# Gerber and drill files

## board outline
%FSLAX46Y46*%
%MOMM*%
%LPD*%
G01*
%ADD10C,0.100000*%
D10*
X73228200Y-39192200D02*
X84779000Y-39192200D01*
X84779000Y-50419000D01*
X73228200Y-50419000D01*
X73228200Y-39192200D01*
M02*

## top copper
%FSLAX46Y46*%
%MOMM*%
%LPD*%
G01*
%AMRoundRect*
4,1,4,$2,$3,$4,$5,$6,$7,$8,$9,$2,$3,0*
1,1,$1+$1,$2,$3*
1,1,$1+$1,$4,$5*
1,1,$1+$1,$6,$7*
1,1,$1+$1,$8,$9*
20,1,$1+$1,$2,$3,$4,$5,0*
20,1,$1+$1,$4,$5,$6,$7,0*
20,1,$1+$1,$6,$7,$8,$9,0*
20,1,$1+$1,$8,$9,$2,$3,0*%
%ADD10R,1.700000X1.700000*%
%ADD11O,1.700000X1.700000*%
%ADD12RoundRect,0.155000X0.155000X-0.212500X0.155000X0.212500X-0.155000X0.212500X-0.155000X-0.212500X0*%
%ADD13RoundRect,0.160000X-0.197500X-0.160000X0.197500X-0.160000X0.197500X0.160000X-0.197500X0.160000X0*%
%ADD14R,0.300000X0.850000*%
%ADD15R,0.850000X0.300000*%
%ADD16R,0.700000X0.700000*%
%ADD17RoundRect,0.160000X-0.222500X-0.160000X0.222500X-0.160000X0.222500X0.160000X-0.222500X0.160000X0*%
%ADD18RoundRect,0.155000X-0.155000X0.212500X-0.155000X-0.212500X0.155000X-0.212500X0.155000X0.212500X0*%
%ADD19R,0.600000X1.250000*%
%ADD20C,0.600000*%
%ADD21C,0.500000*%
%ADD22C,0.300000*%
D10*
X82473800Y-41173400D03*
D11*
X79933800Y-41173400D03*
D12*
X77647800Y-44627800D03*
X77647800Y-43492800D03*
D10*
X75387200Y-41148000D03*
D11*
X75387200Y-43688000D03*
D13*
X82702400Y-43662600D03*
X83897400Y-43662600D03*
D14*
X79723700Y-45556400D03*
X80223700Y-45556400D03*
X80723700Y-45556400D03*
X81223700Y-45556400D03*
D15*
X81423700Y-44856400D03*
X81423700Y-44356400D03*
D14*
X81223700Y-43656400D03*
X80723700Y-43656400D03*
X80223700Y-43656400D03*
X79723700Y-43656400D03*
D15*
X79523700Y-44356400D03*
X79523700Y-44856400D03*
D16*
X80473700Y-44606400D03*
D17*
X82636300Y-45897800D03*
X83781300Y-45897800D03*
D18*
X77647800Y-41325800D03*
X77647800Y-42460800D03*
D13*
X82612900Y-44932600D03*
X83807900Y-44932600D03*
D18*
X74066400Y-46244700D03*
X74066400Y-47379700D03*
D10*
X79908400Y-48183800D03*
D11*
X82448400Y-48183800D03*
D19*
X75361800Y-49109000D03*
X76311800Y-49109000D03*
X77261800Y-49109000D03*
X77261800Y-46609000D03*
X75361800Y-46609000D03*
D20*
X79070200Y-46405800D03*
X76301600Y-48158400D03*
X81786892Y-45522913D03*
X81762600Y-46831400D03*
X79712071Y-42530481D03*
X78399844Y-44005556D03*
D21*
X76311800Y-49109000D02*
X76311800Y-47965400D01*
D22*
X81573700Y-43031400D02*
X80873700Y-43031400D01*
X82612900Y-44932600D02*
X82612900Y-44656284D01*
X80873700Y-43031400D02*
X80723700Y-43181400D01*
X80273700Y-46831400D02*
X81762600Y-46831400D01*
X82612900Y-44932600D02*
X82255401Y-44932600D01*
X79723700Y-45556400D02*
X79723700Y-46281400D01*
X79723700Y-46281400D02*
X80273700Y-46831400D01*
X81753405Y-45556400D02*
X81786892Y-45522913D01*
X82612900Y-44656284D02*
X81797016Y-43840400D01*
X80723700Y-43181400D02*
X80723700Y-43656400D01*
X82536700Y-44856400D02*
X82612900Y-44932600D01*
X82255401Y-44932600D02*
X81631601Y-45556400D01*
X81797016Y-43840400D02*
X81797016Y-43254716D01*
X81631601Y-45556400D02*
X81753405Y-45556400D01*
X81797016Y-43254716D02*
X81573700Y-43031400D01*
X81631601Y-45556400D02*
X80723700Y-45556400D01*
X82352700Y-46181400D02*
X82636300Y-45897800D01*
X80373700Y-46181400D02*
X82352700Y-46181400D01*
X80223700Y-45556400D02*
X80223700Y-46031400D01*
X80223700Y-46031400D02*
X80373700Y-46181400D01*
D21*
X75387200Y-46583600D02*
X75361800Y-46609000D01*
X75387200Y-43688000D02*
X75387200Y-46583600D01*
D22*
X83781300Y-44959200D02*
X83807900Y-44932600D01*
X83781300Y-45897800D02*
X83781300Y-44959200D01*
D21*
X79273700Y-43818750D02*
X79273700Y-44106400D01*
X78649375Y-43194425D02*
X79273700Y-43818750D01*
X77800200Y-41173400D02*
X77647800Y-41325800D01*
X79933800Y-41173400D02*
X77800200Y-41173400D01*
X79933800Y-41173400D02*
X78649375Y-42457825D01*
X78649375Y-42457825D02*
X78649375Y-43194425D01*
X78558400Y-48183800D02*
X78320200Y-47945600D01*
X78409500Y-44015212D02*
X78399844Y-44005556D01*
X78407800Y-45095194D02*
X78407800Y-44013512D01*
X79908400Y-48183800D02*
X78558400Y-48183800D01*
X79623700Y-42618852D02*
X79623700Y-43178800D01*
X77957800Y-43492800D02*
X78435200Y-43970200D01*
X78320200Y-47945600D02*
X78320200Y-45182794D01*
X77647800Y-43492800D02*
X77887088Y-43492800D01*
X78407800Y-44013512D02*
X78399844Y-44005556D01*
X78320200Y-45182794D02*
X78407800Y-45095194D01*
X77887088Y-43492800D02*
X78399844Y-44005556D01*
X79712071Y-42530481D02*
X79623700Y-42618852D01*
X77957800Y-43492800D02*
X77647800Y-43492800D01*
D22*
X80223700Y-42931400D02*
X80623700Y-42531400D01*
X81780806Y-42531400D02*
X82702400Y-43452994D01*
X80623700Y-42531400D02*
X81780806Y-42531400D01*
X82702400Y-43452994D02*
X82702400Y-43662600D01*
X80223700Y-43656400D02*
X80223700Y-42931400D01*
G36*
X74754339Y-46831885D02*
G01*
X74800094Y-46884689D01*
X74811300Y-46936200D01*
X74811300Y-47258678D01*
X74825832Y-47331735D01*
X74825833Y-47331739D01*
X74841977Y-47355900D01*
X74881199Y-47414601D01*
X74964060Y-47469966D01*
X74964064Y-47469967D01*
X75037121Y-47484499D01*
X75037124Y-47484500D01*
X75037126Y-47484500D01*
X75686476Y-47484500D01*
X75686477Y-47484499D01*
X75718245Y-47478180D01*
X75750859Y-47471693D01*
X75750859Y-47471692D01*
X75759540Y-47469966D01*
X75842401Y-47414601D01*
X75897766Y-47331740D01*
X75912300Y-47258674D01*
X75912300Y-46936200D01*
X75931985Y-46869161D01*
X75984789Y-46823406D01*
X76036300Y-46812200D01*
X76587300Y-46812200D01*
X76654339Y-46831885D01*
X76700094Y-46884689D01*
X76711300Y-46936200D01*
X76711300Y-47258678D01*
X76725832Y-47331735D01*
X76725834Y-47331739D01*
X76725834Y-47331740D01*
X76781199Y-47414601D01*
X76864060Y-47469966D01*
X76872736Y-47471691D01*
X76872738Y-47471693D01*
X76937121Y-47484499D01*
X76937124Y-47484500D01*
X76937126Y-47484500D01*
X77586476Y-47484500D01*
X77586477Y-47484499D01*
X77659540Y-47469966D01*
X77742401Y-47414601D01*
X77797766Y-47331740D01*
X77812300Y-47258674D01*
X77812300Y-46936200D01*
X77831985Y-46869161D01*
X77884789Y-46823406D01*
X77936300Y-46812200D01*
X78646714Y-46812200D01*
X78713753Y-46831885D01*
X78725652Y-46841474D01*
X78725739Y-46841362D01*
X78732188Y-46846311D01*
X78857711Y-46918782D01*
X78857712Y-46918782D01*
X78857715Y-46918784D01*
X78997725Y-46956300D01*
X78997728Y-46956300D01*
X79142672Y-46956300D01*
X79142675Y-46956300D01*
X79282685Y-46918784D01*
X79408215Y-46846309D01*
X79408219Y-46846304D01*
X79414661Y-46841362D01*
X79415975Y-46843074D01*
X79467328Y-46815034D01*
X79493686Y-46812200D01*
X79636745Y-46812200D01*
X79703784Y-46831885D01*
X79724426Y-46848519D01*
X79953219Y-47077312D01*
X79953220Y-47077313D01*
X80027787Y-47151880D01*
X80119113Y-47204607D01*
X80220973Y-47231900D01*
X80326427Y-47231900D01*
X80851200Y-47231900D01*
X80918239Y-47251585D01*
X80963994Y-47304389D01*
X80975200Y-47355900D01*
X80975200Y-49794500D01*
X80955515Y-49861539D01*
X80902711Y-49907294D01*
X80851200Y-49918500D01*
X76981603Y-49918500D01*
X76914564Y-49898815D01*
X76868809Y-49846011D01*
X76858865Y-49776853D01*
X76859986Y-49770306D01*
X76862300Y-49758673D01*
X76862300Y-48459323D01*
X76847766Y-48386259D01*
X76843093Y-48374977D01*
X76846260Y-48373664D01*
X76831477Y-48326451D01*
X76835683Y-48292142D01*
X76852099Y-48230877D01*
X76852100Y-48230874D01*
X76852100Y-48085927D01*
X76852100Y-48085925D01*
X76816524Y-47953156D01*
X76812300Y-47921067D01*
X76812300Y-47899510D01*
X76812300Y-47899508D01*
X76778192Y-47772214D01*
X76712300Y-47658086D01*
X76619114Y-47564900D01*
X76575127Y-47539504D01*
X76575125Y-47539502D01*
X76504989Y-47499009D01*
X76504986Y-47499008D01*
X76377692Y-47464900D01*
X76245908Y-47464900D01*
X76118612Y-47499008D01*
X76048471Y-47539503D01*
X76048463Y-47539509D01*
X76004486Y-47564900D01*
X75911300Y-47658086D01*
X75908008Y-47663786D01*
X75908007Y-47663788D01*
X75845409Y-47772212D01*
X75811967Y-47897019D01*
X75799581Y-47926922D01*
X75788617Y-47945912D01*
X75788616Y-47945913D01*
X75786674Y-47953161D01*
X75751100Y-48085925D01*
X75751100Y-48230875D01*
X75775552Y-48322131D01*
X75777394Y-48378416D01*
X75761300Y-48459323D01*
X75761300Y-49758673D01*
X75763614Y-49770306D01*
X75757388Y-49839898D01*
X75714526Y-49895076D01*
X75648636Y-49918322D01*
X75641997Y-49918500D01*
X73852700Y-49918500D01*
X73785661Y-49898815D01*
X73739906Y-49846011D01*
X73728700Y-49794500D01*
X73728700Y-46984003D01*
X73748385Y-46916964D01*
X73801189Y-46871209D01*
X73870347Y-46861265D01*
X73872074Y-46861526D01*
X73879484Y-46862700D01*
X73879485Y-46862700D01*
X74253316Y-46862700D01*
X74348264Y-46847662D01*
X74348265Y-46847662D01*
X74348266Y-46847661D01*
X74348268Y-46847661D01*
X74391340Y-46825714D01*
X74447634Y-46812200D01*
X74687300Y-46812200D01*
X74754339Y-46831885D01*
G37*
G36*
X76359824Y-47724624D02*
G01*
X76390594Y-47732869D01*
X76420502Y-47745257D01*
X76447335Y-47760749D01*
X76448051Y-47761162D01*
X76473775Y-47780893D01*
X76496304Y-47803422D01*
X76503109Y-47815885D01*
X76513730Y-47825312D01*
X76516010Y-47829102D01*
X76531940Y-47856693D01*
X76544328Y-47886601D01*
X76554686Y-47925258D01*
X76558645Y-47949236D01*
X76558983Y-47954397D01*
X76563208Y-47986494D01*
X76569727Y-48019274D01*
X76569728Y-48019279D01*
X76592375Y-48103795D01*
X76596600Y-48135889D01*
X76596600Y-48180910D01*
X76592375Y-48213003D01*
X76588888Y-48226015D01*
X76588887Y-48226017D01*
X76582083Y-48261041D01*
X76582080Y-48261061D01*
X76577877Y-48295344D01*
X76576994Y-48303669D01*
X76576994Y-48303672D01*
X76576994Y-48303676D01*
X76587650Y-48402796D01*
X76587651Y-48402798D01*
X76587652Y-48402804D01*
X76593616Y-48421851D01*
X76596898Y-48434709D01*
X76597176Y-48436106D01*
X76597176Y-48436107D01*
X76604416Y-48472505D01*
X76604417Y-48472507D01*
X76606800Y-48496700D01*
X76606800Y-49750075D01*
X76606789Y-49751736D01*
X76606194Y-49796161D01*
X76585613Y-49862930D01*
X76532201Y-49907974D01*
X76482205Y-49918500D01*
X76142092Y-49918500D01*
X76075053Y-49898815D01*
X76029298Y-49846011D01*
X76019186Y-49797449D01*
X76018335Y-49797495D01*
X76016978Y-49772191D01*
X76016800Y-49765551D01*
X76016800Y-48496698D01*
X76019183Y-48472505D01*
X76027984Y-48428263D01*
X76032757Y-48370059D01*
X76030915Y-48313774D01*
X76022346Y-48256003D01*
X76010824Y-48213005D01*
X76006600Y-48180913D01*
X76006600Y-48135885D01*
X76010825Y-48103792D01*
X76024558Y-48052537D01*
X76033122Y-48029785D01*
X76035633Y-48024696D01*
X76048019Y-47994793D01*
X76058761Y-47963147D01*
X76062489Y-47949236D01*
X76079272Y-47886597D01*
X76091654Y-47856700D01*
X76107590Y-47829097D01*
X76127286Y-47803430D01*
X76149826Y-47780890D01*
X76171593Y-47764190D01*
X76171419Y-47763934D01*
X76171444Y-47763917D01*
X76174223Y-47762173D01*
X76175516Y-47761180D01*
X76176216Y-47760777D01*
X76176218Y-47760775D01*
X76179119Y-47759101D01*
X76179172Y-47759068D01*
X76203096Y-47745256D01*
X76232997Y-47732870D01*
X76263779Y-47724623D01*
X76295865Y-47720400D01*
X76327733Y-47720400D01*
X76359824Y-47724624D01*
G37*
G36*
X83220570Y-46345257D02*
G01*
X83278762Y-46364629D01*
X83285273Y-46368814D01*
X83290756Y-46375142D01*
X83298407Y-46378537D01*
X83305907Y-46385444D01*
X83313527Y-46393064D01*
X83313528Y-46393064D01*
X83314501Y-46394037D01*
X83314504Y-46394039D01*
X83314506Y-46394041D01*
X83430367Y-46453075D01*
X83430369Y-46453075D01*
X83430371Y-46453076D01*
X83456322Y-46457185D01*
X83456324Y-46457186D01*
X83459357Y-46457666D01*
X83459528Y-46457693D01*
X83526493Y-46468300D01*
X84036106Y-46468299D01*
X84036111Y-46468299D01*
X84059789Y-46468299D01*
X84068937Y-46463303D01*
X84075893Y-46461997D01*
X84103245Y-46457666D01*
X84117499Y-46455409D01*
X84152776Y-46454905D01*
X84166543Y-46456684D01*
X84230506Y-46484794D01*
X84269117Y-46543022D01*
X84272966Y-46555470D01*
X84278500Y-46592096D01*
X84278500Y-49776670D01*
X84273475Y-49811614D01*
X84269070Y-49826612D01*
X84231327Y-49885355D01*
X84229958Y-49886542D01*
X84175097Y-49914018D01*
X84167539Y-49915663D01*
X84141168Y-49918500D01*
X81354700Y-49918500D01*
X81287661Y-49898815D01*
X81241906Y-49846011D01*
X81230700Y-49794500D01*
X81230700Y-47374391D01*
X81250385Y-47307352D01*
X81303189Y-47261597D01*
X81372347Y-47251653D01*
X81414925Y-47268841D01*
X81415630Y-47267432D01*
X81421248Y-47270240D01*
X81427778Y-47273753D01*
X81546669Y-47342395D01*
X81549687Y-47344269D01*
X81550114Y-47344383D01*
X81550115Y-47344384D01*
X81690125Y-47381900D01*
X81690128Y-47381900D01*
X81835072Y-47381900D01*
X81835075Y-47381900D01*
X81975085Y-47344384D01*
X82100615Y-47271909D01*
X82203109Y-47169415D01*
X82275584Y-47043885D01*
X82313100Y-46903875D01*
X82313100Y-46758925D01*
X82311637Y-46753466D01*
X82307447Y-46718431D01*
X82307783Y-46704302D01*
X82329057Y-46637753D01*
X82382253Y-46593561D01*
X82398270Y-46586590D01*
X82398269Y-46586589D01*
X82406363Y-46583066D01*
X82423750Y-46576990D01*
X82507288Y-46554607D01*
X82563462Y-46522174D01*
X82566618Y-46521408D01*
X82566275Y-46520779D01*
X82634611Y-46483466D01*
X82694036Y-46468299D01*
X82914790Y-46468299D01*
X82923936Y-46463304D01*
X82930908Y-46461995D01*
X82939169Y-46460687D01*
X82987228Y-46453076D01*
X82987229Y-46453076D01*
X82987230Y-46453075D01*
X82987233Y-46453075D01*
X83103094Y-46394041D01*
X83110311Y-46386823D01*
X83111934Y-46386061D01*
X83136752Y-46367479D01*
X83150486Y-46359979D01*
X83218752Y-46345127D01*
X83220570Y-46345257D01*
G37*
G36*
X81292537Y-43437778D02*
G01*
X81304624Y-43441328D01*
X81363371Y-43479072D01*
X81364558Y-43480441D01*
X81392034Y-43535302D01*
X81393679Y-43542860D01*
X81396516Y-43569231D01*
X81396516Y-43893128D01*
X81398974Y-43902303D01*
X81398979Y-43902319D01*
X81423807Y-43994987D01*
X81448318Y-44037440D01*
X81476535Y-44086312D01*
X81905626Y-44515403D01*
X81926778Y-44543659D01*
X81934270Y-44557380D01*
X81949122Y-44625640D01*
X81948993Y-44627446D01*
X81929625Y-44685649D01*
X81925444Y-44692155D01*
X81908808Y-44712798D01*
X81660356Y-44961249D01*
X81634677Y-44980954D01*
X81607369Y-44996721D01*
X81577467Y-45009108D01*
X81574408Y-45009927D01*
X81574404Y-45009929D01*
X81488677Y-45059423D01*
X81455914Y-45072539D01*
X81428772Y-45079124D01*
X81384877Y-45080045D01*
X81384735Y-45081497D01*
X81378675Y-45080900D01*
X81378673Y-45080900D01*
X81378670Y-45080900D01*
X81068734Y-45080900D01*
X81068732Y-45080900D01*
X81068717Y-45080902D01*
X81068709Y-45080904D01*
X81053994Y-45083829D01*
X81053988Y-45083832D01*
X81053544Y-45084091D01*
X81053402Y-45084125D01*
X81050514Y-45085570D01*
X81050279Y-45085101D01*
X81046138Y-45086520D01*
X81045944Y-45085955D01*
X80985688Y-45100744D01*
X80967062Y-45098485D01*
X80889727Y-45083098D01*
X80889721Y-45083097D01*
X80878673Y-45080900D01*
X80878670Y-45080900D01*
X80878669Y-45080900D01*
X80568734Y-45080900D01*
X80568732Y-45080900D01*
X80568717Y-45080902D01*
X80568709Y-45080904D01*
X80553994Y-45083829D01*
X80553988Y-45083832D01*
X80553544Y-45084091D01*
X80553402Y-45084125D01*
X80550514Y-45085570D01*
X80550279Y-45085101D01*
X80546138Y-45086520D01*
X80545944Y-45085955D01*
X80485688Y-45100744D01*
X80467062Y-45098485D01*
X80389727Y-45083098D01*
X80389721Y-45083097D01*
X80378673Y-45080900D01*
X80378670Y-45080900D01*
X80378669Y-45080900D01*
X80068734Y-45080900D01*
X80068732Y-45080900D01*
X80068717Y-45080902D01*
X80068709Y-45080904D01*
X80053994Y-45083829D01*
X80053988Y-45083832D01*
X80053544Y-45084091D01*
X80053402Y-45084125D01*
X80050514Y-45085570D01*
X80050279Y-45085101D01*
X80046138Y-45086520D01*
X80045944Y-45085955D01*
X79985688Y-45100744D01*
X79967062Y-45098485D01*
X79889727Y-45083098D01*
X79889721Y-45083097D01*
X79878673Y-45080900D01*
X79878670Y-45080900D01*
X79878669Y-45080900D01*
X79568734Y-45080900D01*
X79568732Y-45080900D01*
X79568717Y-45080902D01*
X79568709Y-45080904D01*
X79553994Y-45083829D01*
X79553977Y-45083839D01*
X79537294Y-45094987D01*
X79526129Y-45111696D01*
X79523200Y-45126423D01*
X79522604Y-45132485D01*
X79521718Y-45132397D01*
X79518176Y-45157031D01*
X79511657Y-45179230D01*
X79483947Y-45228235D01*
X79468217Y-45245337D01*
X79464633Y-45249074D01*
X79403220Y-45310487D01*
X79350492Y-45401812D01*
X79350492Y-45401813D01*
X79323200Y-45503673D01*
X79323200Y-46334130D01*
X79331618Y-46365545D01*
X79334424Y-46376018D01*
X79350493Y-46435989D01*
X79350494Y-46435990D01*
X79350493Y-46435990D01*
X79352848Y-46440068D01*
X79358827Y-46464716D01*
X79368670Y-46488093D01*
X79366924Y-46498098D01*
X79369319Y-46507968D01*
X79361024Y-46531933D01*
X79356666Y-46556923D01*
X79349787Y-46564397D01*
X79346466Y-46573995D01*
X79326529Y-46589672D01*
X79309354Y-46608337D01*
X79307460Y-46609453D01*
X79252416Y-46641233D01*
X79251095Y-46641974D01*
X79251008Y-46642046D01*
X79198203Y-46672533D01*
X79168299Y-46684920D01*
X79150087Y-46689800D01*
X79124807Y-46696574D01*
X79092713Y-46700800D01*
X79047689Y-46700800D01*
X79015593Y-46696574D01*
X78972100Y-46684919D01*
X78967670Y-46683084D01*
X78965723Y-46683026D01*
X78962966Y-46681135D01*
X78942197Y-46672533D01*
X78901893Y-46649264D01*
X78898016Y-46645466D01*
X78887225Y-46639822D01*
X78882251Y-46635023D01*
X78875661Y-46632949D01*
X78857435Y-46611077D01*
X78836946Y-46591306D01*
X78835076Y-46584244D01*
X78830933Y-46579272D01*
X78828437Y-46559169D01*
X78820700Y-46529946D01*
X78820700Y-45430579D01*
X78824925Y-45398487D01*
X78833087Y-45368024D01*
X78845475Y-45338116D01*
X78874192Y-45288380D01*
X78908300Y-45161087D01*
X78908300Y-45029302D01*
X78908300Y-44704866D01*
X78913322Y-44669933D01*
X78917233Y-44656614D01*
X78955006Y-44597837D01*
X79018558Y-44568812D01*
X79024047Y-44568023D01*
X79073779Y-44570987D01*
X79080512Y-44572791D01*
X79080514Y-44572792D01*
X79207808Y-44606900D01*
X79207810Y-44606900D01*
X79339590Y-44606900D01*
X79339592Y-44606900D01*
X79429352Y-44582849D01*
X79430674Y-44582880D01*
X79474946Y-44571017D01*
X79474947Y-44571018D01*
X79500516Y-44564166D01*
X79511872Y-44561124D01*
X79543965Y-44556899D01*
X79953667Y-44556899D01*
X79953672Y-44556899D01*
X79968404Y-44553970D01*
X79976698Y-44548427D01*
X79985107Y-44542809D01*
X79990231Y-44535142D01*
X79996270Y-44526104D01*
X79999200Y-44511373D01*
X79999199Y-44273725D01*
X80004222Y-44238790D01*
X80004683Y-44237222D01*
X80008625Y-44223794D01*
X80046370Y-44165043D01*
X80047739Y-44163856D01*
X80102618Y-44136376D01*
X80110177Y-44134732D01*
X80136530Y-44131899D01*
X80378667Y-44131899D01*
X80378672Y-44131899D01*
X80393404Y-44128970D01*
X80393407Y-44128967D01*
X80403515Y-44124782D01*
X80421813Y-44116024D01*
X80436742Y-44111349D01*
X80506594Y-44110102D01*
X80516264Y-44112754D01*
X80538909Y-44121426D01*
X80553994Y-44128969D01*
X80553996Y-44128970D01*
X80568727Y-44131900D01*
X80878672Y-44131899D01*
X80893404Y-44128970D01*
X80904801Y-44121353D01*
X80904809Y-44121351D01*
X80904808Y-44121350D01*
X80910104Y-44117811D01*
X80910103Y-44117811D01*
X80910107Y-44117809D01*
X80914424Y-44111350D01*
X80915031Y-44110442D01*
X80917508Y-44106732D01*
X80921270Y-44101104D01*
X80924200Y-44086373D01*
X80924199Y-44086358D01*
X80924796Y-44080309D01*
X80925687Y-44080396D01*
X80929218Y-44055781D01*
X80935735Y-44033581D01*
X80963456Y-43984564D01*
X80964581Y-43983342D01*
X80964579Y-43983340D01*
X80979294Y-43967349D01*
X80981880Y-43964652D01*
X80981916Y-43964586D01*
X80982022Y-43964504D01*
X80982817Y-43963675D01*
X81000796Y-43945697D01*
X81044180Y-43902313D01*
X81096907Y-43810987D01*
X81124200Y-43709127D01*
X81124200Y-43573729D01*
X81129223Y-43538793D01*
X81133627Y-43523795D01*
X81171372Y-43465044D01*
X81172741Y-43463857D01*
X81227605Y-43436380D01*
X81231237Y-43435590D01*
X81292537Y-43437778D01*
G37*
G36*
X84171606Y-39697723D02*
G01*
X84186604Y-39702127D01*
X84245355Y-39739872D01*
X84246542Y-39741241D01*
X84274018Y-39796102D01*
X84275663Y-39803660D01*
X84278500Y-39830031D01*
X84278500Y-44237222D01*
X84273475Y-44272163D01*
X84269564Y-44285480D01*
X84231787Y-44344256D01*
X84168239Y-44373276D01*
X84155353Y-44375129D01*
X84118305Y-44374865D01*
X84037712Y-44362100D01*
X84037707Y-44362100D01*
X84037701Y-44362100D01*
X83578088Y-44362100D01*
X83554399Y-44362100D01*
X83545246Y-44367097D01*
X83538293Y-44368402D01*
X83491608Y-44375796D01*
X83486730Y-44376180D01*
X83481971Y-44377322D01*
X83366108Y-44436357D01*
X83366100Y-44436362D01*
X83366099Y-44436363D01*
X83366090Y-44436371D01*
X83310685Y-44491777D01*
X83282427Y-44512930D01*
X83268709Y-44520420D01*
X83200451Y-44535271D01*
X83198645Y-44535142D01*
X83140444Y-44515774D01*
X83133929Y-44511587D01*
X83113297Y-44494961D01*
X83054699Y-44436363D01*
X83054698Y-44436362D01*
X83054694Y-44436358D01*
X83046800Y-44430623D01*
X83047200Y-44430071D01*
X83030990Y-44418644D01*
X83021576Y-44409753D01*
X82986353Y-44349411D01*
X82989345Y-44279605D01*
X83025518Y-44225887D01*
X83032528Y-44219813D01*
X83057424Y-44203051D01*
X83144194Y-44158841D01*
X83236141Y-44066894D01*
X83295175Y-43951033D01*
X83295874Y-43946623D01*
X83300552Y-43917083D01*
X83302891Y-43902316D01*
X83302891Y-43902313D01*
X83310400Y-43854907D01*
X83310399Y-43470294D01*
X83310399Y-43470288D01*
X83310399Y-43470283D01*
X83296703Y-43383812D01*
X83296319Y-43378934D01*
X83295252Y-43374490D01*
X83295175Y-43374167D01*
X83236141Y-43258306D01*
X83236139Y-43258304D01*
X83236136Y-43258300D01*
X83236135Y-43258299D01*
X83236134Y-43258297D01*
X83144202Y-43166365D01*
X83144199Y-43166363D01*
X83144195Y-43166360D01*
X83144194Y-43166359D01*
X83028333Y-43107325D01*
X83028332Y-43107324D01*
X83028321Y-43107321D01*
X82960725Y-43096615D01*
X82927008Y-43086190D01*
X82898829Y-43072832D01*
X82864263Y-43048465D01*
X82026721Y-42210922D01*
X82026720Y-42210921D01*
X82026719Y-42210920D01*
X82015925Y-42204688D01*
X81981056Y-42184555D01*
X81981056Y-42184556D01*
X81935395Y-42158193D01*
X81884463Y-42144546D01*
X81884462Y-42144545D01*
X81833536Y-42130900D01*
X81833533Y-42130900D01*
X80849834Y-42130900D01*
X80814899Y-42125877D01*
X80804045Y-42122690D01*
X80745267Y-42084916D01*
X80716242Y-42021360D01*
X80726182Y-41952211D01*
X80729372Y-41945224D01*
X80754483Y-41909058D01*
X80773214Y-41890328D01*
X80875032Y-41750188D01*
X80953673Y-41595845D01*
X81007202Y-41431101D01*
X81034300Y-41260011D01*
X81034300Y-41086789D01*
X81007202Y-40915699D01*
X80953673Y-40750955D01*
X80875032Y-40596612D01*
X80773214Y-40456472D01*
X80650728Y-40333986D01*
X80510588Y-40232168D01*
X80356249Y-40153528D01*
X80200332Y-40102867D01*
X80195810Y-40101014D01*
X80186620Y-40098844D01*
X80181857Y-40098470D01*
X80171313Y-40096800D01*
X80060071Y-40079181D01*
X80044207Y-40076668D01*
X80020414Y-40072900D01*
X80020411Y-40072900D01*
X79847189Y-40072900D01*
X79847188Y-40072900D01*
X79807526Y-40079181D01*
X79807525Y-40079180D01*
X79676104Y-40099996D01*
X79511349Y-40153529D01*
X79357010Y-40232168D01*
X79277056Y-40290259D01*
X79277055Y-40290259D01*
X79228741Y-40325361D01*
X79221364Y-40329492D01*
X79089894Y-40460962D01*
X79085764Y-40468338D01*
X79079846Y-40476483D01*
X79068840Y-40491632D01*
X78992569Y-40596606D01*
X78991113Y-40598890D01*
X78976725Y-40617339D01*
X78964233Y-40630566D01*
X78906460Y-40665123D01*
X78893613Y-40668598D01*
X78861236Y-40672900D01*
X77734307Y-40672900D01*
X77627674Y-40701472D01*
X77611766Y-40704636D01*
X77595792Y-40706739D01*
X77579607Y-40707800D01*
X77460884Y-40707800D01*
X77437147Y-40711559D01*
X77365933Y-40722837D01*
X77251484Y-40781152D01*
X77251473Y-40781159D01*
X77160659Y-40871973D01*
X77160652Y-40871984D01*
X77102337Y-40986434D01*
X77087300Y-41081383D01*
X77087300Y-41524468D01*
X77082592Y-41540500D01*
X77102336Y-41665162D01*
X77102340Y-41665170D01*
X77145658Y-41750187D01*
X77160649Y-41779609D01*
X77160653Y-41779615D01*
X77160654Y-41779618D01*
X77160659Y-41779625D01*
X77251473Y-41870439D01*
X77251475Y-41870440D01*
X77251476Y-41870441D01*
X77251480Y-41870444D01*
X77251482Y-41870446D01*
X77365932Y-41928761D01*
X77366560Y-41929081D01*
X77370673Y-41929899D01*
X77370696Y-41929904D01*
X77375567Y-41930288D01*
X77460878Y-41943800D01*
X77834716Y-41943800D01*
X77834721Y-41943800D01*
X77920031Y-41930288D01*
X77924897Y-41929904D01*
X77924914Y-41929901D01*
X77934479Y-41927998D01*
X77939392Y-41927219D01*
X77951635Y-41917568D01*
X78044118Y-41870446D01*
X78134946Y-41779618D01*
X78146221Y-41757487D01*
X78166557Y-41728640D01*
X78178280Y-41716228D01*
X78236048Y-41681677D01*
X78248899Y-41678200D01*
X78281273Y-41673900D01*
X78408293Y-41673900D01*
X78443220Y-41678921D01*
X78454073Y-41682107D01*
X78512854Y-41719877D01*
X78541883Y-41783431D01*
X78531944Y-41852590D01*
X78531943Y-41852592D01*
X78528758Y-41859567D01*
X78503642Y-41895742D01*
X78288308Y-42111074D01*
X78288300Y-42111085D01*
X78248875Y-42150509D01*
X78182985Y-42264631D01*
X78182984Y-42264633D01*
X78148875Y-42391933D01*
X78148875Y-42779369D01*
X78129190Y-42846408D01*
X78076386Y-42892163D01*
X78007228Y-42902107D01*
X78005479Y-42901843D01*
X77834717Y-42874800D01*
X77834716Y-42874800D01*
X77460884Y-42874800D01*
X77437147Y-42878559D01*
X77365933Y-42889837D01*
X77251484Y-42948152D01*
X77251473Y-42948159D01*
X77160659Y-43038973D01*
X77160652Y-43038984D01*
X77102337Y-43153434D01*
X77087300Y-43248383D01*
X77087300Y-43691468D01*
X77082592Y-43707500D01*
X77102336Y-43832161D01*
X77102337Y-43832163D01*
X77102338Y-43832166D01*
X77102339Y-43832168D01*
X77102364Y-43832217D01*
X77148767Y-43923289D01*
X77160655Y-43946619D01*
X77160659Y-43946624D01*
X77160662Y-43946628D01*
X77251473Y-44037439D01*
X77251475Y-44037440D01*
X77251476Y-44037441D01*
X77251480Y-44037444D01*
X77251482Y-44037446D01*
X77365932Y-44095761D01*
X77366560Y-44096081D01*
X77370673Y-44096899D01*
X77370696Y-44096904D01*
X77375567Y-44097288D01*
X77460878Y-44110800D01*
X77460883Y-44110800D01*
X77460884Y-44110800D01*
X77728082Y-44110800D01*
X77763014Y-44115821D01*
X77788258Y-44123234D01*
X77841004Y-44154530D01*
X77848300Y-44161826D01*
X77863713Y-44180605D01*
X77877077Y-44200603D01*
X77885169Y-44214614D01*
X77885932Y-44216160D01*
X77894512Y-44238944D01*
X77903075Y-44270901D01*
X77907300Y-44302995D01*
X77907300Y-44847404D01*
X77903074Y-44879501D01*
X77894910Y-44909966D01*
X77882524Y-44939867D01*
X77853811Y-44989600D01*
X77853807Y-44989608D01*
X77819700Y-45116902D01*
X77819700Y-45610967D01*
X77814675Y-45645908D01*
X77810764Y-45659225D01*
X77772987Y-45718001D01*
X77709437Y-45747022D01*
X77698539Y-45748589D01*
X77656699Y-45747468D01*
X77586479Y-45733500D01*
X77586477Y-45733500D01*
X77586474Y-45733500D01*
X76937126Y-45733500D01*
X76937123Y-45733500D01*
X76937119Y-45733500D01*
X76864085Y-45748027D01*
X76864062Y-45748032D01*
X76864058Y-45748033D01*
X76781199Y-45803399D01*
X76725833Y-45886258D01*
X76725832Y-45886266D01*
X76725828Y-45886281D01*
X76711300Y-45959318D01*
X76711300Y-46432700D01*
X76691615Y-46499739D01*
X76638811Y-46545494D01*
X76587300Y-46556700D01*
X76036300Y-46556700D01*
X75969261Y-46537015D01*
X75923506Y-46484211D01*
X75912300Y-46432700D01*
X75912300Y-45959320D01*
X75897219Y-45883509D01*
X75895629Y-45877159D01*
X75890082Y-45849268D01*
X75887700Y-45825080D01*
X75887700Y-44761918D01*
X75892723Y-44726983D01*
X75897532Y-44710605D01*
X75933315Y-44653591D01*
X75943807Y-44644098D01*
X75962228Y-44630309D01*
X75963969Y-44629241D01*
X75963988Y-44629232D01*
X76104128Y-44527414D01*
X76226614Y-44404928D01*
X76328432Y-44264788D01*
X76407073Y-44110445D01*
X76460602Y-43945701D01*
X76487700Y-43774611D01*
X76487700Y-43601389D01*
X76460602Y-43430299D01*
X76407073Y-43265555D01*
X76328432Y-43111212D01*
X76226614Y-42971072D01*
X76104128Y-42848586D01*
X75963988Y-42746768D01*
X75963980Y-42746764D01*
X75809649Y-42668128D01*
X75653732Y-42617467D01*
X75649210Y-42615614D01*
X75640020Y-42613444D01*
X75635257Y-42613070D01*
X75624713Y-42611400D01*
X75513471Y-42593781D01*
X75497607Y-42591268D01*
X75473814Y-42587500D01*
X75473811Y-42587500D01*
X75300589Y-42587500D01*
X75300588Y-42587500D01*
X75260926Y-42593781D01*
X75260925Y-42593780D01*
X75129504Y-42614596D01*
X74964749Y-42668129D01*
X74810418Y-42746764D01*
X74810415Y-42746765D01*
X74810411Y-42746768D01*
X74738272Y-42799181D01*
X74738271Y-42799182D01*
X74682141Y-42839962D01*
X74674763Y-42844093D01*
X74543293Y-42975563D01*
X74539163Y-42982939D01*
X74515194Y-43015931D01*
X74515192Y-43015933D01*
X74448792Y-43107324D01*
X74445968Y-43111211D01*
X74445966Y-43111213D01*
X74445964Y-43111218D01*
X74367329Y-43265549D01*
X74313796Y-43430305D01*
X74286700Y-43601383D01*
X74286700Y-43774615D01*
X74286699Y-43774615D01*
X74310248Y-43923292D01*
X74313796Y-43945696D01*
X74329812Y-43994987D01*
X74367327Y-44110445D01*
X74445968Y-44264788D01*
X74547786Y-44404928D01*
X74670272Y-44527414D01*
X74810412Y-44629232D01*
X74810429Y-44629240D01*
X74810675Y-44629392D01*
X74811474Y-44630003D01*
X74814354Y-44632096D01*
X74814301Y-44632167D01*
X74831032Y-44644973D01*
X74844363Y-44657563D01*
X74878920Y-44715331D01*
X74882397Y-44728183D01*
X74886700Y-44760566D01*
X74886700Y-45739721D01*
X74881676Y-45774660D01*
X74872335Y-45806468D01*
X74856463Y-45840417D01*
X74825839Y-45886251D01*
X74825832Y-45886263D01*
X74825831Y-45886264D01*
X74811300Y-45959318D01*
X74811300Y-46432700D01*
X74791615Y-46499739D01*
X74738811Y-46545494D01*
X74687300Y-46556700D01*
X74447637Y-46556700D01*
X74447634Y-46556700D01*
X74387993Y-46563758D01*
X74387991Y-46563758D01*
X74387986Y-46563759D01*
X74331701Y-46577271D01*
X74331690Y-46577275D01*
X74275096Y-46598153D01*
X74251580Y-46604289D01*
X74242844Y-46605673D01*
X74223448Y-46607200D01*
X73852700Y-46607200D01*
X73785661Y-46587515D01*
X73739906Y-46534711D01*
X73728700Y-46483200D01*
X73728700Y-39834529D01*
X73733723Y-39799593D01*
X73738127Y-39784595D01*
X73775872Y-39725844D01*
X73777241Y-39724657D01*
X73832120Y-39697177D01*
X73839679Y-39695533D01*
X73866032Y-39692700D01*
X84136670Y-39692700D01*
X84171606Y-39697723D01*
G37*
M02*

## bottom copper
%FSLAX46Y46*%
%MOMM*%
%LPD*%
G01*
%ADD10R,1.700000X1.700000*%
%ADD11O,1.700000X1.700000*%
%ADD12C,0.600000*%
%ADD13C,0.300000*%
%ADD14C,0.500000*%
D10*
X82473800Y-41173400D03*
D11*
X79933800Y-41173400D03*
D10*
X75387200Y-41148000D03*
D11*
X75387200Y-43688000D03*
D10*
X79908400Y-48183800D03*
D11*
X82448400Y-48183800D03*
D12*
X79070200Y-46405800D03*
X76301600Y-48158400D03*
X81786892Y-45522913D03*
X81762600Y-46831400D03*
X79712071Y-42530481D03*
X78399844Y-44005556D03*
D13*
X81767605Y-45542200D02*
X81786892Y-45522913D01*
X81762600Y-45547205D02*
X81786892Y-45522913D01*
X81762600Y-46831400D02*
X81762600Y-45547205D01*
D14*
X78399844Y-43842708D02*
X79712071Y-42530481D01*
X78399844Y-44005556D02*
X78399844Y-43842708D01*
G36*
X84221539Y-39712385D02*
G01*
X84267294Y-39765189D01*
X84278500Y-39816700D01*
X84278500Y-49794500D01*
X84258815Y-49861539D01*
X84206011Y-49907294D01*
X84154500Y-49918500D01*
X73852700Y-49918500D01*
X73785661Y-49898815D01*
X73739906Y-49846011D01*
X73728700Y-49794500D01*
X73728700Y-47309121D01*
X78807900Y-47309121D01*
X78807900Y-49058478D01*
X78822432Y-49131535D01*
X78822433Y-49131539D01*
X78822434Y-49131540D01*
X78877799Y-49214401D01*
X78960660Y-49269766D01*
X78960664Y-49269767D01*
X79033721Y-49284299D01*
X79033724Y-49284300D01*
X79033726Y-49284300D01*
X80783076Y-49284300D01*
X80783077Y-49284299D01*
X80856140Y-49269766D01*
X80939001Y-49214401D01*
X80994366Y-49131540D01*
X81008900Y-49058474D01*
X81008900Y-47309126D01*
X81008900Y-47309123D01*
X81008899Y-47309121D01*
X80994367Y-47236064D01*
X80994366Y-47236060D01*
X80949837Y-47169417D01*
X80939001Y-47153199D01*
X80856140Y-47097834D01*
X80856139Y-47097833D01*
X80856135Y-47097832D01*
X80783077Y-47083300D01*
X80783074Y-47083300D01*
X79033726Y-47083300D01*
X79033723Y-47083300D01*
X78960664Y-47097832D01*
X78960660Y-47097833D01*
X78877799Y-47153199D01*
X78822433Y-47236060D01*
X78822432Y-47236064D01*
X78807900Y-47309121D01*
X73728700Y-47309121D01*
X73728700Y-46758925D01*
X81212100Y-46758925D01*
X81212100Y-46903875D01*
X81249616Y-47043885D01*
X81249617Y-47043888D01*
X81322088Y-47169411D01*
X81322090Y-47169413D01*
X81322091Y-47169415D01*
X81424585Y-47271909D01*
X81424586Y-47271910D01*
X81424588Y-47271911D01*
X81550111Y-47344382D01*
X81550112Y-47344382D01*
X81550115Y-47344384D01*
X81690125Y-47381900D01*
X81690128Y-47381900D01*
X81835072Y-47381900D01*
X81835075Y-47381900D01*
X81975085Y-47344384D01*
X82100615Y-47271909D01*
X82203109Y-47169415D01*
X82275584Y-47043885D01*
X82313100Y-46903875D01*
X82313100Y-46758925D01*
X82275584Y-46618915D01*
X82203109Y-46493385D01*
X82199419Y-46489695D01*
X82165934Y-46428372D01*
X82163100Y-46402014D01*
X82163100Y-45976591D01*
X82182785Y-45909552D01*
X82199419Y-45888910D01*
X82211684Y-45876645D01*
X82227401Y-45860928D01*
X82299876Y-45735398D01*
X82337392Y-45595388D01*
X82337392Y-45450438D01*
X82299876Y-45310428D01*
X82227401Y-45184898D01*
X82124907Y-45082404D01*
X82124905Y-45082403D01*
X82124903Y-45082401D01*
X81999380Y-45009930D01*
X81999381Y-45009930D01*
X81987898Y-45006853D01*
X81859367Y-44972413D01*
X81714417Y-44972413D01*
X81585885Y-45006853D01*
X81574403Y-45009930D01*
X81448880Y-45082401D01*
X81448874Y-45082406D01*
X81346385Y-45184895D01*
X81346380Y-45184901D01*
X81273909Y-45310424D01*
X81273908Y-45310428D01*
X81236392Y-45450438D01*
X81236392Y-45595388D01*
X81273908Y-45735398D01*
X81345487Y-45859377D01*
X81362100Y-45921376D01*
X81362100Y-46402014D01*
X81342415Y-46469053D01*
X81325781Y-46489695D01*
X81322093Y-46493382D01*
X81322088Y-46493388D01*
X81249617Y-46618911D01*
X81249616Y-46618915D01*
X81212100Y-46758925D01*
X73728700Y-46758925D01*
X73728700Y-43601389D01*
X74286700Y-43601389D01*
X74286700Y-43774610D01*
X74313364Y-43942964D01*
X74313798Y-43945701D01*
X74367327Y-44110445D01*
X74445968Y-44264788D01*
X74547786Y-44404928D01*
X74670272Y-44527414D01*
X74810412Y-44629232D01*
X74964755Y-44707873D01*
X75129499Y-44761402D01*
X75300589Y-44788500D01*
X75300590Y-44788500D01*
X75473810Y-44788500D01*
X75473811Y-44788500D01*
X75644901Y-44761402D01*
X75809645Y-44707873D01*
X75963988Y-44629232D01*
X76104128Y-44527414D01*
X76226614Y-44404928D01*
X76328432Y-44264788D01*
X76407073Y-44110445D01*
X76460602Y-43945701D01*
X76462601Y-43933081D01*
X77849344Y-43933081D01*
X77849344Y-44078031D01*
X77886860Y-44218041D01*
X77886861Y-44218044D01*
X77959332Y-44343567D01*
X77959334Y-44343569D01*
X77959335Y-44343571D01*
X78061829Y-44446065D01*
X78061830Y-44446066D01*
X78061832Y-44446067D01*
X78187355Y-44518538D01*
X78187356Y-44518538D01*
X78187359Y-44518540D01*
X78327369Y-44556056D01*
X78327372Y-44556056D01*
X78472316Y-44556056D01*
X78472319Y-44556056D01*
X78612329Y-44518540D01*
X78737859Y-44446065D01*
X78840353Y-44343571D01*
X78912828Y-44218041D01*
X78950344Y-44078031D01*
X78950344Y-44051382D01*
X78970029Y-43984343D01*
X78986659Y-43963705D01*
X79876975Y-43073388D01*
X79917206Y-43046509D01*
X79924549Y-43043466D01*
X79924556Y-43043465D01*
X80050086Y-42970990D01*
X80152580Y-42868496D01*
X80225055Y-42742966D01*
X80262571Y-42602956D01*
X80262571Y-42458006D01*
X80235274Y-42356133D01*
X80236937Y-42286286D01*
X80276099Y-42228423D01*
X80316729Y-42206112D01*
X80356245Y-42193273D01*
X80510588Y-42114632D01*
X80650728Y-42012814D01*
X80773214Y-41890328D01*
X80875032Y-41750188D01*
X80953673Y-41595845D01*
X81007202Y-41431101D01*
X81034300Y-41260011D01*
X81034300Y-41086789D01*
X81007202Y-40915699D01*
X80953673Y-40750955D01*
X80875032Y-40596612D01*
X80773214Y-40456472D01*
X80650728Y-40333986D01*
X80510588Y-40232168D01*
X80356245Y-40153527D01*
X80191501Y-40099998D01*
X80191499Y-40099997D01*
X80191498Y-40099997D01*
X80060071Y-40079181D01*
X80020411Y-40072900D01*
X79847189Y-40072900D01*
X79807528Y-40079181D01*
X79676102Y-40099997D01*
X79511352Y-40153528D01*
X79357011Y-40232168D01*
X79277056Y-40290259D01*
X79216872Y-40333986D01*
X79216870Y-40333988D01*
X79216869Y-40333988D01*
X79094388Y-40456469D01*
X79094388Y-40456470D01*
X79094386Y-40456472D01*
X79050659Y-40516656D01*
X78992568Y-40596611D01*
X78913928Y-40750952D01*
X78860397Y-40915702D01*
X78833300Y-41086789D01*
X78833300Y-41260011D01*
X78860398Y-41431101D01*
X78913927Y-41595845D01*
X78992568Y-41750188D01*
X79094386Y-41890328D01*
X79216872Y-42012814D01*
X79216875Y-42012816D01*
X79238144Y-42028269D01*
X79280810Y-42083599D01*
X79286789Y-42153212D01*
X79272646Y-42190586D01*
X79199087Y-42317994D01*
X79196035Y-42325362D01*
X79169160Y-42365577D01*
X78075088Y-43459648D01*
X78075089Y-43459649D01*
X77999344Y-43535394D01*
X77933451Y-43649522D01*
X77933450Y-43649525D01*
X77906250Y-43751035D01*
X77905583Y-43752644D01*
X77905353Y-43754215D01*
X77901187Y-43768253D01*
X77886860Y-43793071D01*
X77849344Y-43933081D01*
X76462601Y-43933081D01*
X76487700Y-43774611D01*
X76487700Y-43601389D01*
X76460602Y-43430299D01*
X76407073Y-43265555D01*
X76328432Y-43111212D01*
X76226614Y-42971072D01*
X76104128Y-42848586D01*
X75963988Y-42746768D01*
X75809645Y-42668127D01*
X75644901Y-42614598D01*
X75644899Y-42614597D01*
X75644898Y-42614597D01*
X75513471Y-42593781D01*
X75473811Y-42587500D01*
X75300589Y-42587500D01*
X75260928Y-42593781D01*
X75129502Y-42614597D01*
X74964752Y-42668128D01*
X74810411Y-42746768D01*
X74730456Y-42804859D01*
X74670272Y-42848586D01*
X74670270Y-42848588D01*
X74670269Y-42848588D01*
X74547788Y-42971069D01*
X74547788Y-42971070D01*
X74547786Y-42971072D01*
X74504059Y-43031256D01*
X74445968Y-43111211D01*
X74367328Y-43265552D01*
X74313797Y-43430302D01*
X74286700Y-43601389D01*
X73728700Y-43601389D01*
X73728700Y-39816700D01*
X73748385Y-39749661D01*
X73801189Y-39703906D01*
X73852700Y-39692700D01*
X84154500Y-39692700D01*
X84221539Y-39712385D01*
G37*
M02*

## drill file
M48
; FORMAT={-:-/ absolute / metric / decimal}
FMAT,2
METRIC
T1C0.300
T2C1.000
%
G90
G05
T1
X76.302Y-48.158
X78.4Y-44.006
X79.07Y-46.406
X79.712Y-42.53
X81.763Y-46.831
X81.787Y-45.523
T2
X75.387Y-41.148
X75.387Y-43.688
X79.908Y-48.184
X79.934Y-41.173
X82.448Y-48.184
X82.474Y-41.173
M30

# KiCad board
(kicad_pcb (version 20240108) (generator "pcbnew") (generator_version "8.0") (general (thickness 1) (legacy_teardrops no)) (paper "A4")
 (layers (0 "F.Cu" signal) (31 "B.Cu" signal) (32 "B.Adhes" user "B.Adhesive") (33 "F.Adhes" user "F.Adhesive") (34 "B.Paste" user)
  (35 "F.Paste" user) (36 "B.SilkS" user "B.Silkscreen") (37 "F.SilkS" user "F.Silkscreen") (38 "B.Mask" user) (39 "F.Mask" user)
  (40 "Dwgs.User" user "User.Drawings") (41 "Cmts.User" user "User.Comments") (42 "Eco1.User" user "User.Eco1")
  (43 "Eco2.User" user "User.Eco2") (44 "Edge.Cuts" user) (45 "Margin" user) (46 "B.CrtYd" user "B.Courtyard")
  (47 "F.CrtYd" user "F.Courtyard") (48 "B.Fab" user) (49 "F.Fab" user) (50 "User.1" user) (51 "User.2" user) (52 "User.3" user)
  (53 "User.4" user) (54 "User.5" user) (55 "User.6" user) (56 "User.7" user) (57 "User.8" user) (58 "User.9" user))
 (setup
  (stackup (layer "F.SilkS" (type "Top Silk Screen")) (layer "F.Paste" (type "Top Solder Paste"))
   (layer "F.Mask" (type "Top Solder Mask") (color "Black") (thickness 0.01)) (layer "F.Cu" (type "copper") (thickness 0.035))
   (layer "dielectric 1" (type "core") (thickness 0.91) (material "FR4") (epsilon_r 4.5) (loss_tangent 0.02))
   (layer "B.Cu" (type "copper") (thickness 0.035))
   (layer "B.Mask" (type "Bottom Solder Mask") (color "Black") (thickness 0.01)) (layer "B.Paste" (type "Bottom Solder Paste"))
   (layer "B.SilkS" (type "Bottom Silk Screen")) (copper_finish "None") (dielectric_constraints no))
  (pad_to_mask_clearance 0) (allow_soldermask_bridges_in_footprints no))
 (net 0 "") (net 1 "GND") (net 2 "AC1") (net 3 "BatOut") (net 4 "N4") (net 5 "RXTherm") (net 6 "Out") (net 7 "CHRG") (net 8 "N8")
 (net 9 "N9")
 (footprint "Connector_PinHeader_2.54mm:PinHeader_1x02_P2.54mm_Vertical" (layer "F.Cu") (at 82.4738 41.1734 -90)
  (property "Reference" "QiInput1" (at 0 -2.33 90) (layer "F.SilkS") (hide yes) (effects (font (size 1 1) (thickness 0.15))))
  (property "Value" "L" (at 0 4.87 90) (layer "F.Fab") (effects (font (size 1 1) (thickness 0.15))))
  (pad "1" thru_hole rect (at 0 0 270) (size 1.7 1.7) (drill 1) (layers "*.Cu" "*.Mask") (remove_unused_layers no) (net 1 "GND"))
  (pad "2" thru_hole oval (at 0 2.54 270) (size 1.7 1.7) (drill 1) (layers "*.Cu" "*.Mask") (remove_unused_layers no) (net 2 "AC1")))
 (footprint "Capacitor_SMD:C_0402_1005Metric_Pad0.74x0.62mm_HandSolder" (layer "F.Cu") (at 77.6478 44.0603 90)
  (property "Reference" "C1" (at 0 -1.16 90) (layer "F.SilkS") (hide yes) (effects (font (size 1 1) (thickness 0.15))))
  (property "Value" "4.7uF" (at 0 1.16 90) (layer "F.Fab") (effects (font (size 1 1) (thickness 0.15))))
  (pad "1" smd roundrect (at -0.5675 0 90) (size 0.735 0.62) (layers "F.Cu" "F.Paste" "F.Mask") (roundrect_rratio 0.25) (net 1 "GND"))
  (pad "2" smd roundrect (at 0.5675 0 90) (size 0.735 0.62) (layers "F.Cu" "F.Paste" "F.Mask") (roundrect_rratio 0.25) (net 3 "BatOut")))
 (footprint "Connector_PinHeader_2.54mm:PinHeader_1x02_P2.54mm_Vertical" (layer "F.Cu") (at 75.3872 41.148)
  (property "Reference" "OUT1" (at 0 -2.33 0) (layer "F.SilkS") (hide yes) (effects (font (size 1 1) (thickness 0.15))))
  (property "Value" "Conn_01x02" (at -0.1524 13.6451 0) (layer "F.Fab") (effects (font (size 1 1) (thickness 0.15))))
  (pad "1" thru_hole rect (at 0 0) (size 1.7 1.7) (drill 1) (layers "*.Cu" "*.Mask") (remove_unused_layers no) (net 1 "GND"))
  (pad "2" thru_hole oval (at 0 2.54) (size 1.7 1.7) (drill 1) (layers "*.Cu" "*.Mask") (remove_unused_layers no) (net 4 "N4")))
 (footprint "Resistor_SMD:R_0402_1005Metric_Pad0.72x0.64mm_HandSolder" (layer "F.Cu") (at 83.2999 43.6626)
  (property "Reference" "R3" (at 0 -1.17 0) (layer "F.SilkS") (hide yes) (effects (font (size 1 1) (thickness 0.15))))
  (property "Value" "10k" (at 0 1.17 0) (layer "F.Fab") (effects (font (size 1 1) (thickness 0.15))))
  (pad "1" smd roundrect (at -0.5975 0) (size 0.715 0.64) (layers "F.Cu" "F.Paste" "F.Mask") (roundrect_rratio 0.25) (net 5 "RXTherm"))
  (pad "2" smd roundrect (at 0.5975 0) (size 0.715 0.64) (layers "F.Cu" "F.Paste" "F.Mask") (roundrect_rratio 0.25) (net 1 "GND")))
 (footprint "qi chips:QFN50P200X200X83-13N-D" (layer "F.Cu") (at 80.4737 44.6064 90)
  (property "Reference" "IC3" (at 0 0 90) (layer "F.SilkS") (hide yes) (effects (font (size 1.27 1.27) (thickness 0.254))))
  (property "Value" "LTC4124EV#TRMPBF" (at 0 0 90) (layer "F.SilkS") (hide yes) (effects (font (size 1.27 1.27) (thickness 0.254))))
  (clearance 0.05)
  (pad "1" smd rect (at -0.95 -0.75 180) (size 0.3 0.85) (layers "F.Cu" "F.Paste" "F.Mask") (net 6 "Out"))
  (pad "2" smd rect (at -0.95 -0.25 180) (size 0.3 0.85) (layers "F.Cu" "F.Paste" "F.Mask") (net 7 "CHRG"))
  (pad "3" smd rect (at -0.95 0.25 180) (size 0.3 0.85) (layers "F.Cu" "F.Paste" "F.Mask") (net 6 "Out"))
  (pad "4" smd rect (at -0.95 0.75 180) (size 0.3 0.85) (layers "F.Cu" "F.Paste" "F.Mask") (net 6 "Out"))
  (pad "5" smd rect (at -0.25 0.95 90) (size 0.3 0.85) (layers "F.Cu" "F.Paste" "F.Mask") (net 1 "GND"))
  (pad "6" smd rect (at 0.25 0.95 90) (size 0.3 0.85) (layers "F.Cu" "F.Paste" "F.Mask") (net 1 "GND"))
  (pad "7" smd rect (at 0.95 0.75 180) (size 0.3 0.85) (layers "F.Cu" "F.Paste" "F.Mask") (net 1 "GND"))
  (pad "8" smd rect (at 0.95 0.25 180) (size 0.3 0.85) (layers "F.Cu" "F.Paste" "F.Mask") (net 6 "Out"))
  (pad "9" smd rect (at 0.95 -0.25 180) (size 0.3 0.85) (layers "F.Cu" "F.Paste" "F.Mask") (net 5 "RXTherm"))
  (pad "10" smd rect (at 0.95 -0.75 180) (size 0.3 0.85) (layers "F.Cu" "F.Paste" "F.Mask") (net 3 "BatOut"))
  (pad "11" smd rect (at 0.25 -0.95 90) (size 0.3 0.85) (layers "F.Cu" "F.Paste" "F.Mask") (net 2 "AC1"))
  (pad "12" smd rect (at -0.25 -0.95 90) (size 0.3 0.85) (layers "F.Cu" "F.Paste" "F.Mask") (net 1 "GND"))
  (pad "13" smd rect (at 0 0 90) (size 0.7 0.7) (layers "F.Cu" "F.Paste" "F.Mask") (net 1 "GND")))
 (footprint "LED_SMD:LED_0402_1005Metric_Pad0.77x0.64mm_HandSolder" (layer "F.Cu") (at 83.2088 45.8978)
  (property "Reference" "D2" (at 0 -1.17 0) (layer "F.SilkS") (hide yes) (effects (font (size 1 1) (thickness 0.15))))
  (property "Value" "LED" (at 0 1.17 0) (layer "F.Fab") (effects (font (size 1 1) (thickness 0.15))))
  (pad "1" smd roundrect (at -0.5725 0) (size 0.765 0.64) (layers "F.Cu" "F.Paste" "F.Mask") (roundrect_rratio 0.25) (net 7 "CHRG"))
  (pad "2" smd roundrect (at 0.5725 0) (size 0.765 0.64) (layers "F.Cu" "F.Paste" "F.Mask") (roundrect_rratio 0.25) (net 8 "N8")))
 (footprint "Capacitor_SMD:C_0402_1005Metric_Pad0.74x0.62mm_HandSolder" (layer "F.Cu") (at 77.6478 41.8933 -90)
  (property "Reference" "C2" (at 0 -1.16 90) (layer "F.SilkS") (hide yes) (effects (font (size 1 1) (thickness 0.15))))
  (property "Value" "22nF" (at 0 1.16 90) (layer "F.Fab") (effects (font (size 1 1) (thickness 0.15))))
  (pad "1" smd roundrect (at -0.5675 0 270) (size 0.735 0.62) (layers "F.Cu" "F.Paste" "F.Mask") (roundrect_rratio 0.25) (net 2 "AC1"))
  (pad "2" smd roundrect (at 0.5675 0 270) (size 0.735 0.62) (layers "F.Cu" "F.Paste" "F.Mask") (roundrect_rratio 0.25) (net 1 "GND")))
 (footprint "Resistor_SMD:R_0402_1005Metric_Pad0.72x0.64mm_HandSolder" (layer "F.Cu") (at 83.2104 44.9326)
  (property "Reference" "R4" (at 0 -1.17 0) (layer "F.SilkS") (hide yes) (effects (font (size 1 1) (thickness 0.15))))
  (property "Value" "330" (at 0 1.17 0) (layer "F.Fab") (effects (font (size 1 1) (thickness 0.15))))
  (pad "1" smd roundrect (at -0.5975 0) (size 0.715 0.64) (layers "F.Cu" "F.Paste" "F.Mask") (roundrect_rratio 0.25) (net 6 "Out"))
  (pad "2" smd roundrect (at 0.5975 0) (size 0.715 0.64) (layers "F.Cu" "F.Paste" "F.Mask") (roundrect_rratio 0.25) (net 8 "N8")))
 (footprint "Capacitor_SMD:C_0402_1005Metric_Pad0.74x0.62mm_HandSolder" (layer "F.Cu") (at 74.0664 46.8122 -90)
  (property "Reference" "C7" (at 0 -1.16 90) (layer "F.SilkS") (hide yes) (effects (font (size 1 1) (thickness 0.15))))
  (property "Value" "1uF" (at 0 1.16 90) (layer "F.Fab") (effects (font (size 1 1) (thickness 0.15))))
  (pad "1" smd roundrect (at -0.5675 0 270) (size 0.735 0.62) (layers "F.Cu" "F.Paste" "F.Mask") (roundrect_rratio 0.25) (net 1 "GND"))
  (pad "2" smd roundrect (at 0.5675 0 270) (size 0.735 0.62) (layers "F.Cu" "F.Paste" "F.Mask") (roundrect_rratio 0.25) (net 3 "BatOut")))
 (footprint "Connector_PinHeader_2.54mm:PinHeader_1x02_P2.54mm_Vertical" (layer "F.Cu") (at 79.9084 48.1838 90)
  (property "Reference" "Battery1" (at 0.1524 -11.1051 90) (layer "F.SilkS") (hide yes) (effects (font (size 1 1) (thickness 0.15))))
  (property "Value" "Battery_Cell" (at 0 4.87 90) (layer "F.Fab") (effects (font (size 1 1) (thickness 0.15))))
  (pad "1" thru_hole rect (at 0 0 90) (size 1.7 1.7) (drill 1) (layers "*.Cu" "*.Mask") (remove_unused_layers no) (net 3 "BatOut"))
  (pad "2" thru_hole oval (at 0 2.54 90) (size 1.7 1.7) (drill 1) (layers "*.Cu" "*.Mask") (remove_unused_layers no) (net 1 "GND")))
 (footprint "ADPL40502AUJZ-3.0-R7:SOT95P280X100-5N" (layer "F.Cu") (at 76.3118 47.859 90)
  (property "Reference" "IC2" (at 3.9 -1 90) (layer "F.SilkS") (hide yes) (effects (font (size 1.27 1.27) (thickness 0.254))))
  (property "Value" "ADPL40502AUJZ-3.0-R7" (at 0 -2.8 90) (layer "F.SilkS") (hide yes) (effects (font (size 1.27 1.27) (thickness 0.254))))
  (pad "1" smd rect (at -1.25 -0.95 180) (size 0.6 1.25) (layers "F.Cu" "F.Paste" "F.Mask") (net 3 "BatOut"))
  (pad "2" smd rect (at -1.25 0 180) (size 0.6 1.25) (layers "F.Cu" "F.Paste" "F.Mask") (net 1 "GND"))
  (pad "3" smd rect (at -1.25 0.95 180) (size 0.6 1.25) (layers "F.Cu" "F.Paste" "F.Mask") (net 3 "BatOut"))
  (pad "4" smd rect (at 1.25 0.95 180) (size 0.6 1.25) (layers "F.Cu" "F.Paste" "F.Mask") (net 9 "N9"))
  (pad "5" smd rect (at 1.25 -0.95 180) (size 0.6 1.25) (layers "F.Cu" "F.Paste" "F.Mask") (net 4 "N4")))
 (gr_rect (start 73.2282 39.1922) (end 84.779 50.419) (stroke (width 0.1) (type default)) (fill none) (layer "Edge.Cuts"))
 (segment (start 76.3118 49.109) (end 76.3118 47.9654) (width 0.5) (layer "F.Cu") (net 1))
 (via (at 79.0702 46.4058) (size 0.6) (drill 0.3) (layers "F.Cu" "B.Cu") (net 1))
 (via (at 76.3016 48.1584) (size 0.6) (drill 0.3) (layers "F.Cu" "B.Cu") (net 1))
 (segment (start 81.5737 43.0314) (end 80.8737 43.0314) (width 0.3) (layer "F.Cu") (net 6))
 (segment (start 82.6129 44.9326) (end 82.6129 44.656284) (width 0.3) (layer "F.Cu") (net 6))
 (segment (start 80.8737 43.0314) (end 80.7237 43.1814) (width 0.3) (layer "F.Cu") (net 6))
 (segment (start 80.2737 46.8314) (end 81.7626 46.8314) (width 0.3) (layer "F.Cu") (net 6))
 (segment (start 82.6129 44.9326) (end 82.255401 44.9326) (width 0.3) (layer "F.Cu") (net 6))
 (segment (start 79.7237 45.5564) (end 79.7237 46.2814) (width 0.3) (layer "F.Cu") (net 6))
 (segment (start 79.7237 46.2814) (end 80.2737 46.8314) (width 0.3) (layer "F.Cu") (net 6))
 (segment (start 81.753405 45.5564) (end 81.786892 45.522913) (width 0.3) (layer "F.Cu") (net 6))
 (segment (start 82.6129 44.656284) (end 81.797016 43.8404) (width 0.3) (layer "F.Cu") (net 6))
 (segment (start 80.7237 43.1814) (end 80.7237 43.6564) (width 0.3) (layer "F.Cu") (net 6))
 (segment (start 82.5367 44.8564) (end 82.6129 44.9326) (width 0.3) (layer "F.Cu") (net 6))
 (segment (start 82.255401 44.9326) (end 81.631601 45.5564) (width 0.3) (layer "F.Cu") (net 6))
 (segment (start 81.797016 43.8404) (end 81.797016 43.254716) (width 0.3) (layer "F.Cu") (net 6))
 (segment (start 81.631601 45.5564) (end 81.753405 45.5564) (width 0.3) (layer "F.Cu") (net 6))
 (segment (start 81.797016 43.254716) (end 81.5737 43.0314) (width 0.3) (layer "F.Cu") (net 6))
 (segment (start 81.631601 45.5564) (end 80.7237 45.5564) (width 0.3) (layer "F.Cu") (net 6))
 (via (at 81.786892 45.522913) (size 0.6) (drill 0.3) (layers "F.Cu" "B.Cu") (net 6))
 (via (at 81.7626 46.8314) (size 0.6) (drill 0.3) (layers "F.Cu" "B.Cu") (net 6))
 (segment (start 81.767605 45.5422) (end 81.786892 45.522913) (width 0.3) (layer "B.Cu") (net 6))
 (segment (start 81.7626 45.547205) (end 81.786892 45.522913) (width 0.3) (layer "B.Cu") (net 6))
 (segment (start 81.7626 46.8314) (end 81.7626 45.547205) (width 0.3) (layer "B.Cu") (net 6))
 (segment (start 82.3527 46.1814) (end 82.6363 45.8978) (width 0.3) (layer "F.Cu") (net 7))
 (segment (start 80.3737 46.1814) (end 82.3527 46.1814) (width 0.3) (layer "F.Cu") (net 7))
 (segment (start 80.2237 45.5564) (end 80.2237 46.0314) (width 0.3) (layer "F.Cu") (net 7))
 (segment (start 80.2237 46.0314) (end 80.3737 46.1814) (width 0.3) (layer "F.Cu") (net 7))
 (segment (start 75.3872 46.5836) (end 75.3618 46.609) (width 0.5) (layer "F.Cu") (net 4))
 (segment (start 75.3872 43.688) (end 75.3872 46.5836) (width 0.5) (layer "F.Cu") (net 4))
 (segment (start 83.7813 44.9592) (end 83.8079 44.9326) (width 0.3) (layer "F.Cu") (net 8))
 (segment (start 83.7813 45.8978) (end 83.7813 44.9592) (width 0.3) (layer "F.Cu") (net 8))
 (segment (start 79.2737 43.81875) (end 79.2737 44.1064) (width 0.5) (layer "F.Cu") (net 2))
 (segment (start 78.649375 43.194425) (end 79.2737 43.81875) (width 0.5) (layer "F.Cu") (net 2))
 (segment (start 77.8002 41.1734) (end 77.6478 41.3258) (width 0.5) (layer "F.Cu") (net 2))
 (segment (start 79.9338 41.1734) (end 77.8002 41.1734) (width 0.5) (layer "F.Cu") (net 2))
 (segment (start 79.9338 41.1734) (end 78.649375 42.457825) (width 0.5) (layer "F.Cu") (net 2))
 (segment (start 78.649375 42.457825) (end 78.649375 43.194425) (width 0.5) (layer "F.Cu") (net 2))
 (segment (start 78.5584 48.1838) (end 78.3202 47.9456) (width 0.5) (layer "F.Cu") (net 3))
 (segment (start 78.4095 44.015212) (end 78.399844 44.005556) (width 0.5) (layer "F.Cu") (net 3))
 (segment (start 78.4078 45.095194) (end 78.4078 44.013512) (width 0.5) (layer "F.Cu") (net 3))
 (segment (start 79.9084 48.1838) (end 78.5584 48.1838) (width 0.5) (layer "F.Cu") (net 3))
 (segment (start 79.6237 42.618852) (end 79.6237 43.1788) (width 0.5) (layer "F.Cu") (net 3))
 (segment (start 77.9578 43.4928) (end 78.4352 43.9702) (width 0.5) (layer "F.Cu") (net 3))
 (segment (start 78.3202 47.9456) (end 78.3202 45.182794) (width 0.5) (layer "F.Cu") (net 3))
 (segment (start 77.6478 43.4928) (end 77.887088 43.4928) (width 0.5) (layer "F.Cu") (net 3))
 (segment (start 78.4078 44.013512) (end 78.399844 44.005556) (width 0.5) (layer "F.Cu") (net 3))
 (segment (start 78.3202 45.182794) (end 78.4078 45.095194) (width 0.5) (layer "F.Cu") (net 3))
 (segment (start 77.887088 43.4928) (end 78.399844 44.005556) (width 0.5) (layer "F.Cu") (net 3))
 (segment (start 79.712071 42.530481) (end 79.6237 42.618852) (width 0.5) (layer "F.Cu") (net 3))
 (segment (start 77.9578 43.4928) (end 77.6478 43.4928) (width 0.5) (layer "F.Cu") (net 3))
 (via (at 79.712071 42.530481) (size 0.6) (drill 0.3) (layers "F.Cu" "B.Cu") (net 3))
 (via (at 78.399844 44.005556) (size 0.6) (drill 0.3) (layers "F.Cu" "B.Cu") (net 3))
 (segment (start 78.399844 43.842708) (end 79.712071 42.530481) (width 0.5) (layer "B.Cu") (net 3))
 (segment (start 78.399844 44.005556) (end 78.399844 43.842708) (width 0.5) (layer "B.Cu") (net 3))
 (segment (start 80.2237 42.9314) (end 80.6237 42.5314) (width 0.3) (layer "F.Cu") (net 5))
 (segment (start 81.780806 42.5314) (end 82.7024 43.452994) (width 0.3) (layer "F.Cu") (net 5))
 (segment (start 80.6237 42.5314) (end 81.780806 42.5314) (width 0.3) (layer "F.Cu") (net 5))
 (segment (start 82.7024 43.452994) (end 82.7024 43.6626) (width 0.3) (layer "F.Cu") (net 5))
 (segment (start 80.2237 43.6564) (end 80.2237 42.9314) (width 0.3) (layer "F.Cu") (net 5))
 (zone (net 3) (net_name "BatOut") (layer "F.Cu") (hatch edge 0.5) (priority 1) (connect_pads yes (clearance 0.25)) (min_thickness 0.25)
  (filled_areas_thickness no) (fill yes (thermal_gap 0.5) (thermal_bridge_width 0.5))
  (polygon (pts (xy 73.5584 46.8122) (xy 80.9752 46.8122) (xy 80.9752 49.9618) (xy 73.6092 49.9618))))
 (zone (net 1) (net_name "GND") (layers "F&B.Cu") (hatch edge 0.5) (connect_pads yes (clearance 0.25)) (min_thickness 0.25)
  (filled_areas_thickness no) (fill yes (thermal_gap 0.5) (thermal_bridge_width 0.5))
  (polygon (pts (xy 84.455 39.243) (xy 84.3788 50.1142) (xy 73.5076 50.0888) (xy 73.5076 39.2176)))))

